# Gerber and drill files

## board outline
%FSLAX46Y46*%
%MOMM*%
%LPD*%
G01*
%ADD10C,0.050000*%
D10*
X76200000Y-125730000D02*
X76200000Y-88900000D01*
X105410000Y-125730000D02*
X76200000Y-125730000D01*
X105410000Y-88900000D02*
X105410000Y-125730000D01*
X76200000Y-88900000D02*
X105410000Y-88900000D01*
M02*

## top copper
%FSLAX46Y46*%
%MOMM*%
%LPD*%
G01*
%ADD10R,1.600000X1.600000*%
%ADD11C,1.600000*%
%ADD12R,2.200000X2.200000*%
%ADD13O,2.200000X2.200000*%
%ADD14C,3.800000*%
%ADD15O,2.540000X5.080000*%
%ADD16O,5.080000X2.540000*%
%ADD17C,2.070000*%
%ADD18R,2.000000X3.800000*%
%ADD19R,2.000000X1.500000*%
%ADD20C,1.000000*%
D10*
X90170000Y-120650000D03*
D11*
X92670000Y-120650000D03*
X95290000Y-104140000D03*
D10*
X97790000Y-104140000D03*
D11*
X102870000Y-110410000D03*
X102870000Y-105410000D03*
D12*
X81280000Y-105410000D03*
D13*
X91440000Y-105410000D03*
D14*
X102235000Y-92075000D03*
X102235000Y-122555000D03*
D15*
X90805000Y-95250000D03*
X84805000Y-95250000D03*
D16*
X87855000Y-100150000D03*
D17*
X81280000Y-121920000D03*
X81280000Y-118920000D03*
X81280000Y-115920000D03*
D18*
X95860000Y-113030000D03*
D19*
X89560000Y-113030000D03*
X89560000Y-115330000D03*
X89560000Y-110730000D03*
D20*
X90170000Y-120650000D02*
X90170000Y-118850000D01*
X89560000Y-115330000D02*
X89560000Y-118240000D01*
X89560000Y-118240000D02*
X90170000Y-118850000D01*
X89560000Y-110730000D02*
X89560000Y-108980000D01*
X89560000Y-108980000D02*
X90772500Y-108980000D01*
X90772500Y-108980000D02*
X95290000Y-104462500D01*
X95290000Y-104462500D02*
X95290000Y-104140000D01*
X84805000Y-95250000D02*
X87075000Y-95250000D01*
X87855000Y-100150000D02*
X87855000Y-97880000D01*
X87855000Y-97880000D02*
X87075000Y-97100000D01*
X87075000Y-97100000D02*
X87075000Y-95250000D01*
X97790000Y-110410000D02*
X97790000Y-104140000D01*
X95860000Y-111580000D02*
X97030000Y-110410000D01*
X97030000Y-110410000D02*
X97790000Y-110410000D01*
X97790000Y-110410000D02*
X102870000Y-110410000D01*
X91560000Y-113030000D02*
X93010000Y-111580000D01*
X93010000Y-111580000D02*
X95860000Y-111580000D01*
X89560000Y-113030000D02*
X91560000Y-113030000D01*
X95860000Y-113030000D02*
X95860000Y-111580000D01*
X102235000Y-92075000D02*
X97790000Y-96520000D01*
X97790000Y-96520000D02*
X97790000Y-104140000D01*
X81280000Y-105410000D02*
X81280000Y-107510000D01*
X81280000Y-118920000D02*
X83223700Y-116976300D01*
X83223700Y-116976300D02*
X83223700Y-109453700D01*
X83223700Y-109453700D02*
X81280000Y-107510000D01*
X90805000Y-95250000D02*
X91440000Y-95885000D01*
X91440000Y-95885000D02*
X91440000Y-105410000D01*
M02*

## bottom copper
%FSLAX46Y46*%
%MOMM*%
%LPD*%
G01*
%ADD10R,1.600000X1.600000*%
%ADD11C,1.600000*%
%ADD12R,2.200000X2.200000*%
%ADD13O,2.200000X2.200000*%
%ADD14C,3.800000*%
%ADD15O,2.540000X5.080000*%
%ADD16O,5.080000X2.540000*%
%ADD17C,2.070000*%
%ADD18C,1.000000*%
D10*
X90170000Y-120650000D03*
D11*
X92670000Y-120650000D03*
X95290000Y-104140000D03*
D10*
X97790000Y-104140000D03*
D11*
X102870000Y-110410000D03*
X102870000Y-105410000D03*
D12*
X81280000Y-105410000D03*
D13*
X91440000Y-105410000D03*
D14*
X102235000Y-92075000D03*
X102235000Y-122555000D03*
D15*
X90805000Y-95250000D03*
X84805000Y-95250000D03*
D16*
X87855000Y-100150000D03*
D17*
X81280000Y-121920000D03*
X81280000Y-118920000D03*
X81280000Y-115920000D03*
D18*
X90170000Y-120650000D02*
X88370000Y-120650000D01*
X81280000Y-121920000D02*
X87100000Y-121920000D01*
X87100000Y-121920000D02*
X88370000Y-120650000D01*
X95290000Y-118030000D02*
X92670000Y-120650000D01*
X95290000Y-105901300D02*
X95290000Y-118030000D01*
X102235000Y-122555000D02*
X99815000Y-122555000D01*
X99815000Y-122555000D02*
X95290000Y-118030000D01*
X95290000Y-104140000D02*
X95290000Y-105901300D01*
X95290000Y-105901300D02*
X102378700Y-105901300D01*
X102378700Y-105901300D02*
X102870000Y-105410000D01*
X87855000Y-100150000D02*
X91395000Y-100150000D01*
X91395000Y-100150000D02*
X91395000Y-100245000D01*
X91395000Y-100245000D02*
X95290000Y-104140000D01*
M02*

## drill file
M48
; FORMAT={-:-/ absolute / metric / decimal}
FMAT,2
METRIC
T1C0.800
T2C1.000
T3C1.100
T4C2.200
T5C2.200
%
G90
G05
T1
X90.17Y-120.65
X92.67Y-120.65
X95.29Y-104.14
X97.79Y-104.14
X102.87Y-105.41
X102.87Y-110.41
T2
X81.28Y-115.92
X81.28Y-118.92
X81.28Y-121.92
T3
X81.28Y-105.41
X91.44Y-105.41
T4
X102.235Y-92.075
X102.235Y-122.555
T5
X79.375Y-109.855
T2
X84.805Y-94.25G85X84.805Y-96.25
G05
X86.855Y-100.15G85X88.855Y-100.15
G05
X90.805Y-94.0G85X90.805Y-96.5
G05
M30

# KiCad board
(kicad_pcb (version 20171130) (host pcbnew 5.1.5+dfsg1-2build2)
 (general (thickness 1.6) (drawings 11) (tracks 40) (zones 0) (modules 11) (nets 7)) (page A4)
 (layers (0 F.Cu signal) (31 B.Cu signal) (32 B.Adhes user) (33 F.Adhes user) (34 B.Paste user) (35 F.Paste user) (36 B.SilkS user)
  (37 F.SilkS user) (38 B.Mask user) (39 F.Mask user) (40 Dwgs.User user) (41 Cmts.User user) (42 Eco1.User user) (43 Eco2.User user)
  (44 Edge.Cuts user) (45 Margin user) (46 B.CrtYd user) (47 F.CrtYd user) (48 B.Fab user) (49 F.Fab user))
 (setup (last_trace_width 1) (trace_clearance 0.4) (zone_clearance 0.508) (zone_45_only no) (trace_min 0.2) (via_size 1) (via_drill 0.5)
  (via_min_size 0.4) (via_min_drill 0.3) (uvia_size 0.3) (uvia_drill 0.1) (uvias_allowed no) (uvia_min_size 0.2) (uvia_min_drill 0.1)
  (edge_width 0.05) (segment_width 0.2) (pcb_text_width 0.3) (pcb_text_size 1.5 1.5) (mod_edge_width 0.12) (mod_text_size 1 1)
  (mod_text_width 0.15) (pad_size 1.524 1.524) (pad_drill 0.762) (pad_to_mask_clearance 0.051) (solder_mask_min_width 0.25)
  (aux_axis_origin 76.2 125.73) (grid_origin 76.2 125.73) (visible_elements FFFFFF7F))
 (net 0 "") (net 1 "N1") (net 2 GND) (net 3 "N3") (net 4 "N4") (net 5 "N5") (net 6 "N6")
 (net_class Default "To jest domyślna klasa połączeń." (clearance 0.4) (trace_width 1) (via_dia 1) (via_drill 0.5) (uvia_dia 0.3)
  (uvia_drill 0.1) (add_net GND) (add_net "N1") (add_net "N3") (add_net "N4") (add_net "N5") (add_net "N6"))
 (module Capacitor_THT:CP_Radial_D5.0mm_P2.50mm (layer F.Cu) (at 90.17 120.65)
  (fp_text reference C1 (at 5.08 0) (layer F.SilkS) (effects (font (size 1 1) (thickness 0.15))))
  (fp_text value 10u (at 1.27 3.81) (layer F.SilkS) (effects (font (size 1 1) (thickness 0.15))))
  (pad 1 thru_hole rect (at 0 0) (size 1.6 1.6) (drill 0.8) (layers *.Cu *.Mask) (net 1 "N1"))
  (pad 2 thru_hole circle (at 2.5 0) (size 1.6 1.6) (drill 0.8) (layers *.Cu *.Mask) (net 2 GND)))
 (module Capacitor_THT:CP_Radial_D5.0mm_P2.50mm (layer F.Cu) (at 97.79 104.14 180)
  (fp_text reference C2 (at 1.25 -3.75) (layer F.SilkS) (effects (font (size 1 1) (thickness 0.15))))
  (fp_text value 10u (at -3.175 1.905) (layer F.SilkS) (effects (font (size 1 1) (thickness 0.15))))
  (pad 2 thru_hole circle (at 2.5 0 180) (size 1.6 1.6) (drill 0.8) (layers *.Cu *.Mask) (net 2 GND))
  (pad 1 thru_hole rect (at 0 0 180) (size 1.6 1.6) (drill 0.8) (layers *.Cu *.Mask) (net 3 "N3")))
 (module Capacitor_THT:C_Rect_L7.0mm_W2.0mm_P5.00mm (layer F.Cu) (at 102.87 110.41 90)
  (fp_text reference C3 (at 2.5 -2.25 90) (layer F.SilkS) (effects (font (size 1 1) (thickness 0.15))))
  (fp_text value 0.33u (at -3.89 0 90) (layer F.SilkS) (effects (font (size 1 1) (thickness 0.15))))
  (pad 1 thru_hole circle (at 0 0 90) (size 1.6 1.6) (drill 0.8) (layers *.Cu *.Mask) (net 3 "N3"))
  (pad 2 thru_hole circle (at 5 0 90) (size 1.6 1.6) (drill 0.8) (layers *.Cu *.Mask) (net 2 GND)))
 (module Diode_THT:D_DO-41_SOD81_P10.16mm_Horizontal (layer F.Cu) (at 81.28 105.41)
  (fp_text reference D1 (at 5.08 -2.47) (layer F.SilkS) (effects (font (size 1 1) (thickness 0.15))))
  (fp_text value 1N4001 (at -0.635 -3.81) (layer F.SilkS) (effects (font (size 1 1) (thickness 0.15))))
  (pad 1 thru_hole rect (at 0 0) (size 2.2 2.2) (drill 1.1) (layers *.Cu *.Mask) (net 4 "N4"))
  (pad 2 thru_hole oval (at 10.16 0) (size 2.2 2.2) (drill 1.1) (layers *.Cu *.Mask) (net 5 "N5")))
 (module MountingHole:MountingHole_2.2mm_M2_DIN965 (layer F.Cu) (at 79.375 109.855)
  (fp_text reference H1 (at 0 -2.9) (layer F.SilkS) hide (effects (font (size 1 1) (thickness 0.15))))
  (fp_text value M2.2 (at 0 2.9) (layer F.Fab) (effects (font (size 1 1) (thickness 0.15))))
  (pad 1 np_thru_hole circle (at 0 0) (size 2.2 2.2) (drill 2.2) (layers *.Cu *.Mask)))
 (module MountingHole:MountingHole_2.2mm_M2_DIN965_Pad (layer F.Cu) (at 102.235 92.075)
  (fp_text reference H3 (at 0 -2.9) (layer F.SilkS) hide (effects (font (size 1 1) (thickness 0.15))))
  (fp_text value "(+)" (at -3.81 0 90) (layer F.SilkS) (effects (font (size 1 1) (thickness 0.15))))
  (pad 1 thru_hole circle (at 0 0) (size 3.8 3.8) (drill 2.2) (layers *.Cu *.Mask) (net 3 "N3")))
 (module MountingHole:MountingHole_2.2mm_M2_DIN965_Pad (layer F.Cu) (at 102.235 122.555)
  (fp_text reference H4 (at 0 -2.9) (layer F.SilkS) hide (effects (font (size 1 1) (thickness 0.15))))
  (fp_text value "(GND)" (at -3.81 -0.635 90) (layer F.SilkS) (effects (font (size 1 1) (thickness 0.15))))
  (pad 1 thru_hole circle (at 0 0) (size 3.8 3.8) (drill 2.2) (layers *.Cu *.Mask) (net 2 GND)))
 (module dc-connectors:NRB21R (layer F.Cu) (at 90.805 95.25 270)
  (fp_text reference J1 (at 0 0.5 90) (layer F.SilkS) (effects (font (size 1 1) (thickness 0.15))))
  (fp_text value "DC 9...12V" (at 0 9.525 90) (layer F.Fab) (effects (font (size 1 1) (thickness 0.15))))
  (pad 1 thru_hole oval (at 0 0 270) (size 5.08 2.54) (drill oval 3.5 1) (layers *.Cu *.Mask) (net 5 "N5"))
  (pad 2 thru_hole oval (at 0 6 270) (size 5.08 2.54) (drill oval 3 1) (layers *.Cu *.Mask) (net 2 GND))
  (pad 3 thru_hole oval (at 4.9 2.95) (size 5.08 2.54) (drill oval 3 1) (layers *.Cu *.Mask) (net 2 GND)))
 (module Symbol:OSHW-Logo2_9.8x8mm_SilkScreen (layer F.Cu) (at 98.425 97.155)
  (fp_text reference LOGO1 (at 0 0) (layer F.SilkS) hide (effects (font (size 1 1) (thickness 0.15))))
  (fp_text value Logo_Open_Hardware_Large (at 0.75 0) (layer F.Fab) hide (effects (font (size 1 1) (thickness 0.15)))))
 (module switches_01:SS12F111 (layer F.Cu) (at 81.28 118.92 90)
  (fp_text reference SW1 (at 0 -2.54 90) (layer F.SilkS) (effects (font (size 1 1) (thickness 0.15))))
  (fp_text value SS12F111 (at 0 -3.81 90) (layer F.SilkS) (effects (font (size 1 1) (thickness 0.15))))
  (pad 1 thru_hole circle (at -3 0 90) (size 2.07 2.07) (drill 1) (layers *.Cu *.Mask) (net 1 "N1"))
  (pad 2 thru_hole circle (at 0 0 90) (size 2.07 2.07) (drill 1) (layers *.Cu *.Mask) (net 4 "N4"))
  (pad 3 thru_hole circle (at 3 0 90) (size 2.07 2.07) (drill 1) (layers *.Cu *.Mask) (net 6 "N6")))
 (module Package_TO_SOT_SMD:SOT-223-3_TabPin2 (layer F.Cu) (at 92.71 113.03)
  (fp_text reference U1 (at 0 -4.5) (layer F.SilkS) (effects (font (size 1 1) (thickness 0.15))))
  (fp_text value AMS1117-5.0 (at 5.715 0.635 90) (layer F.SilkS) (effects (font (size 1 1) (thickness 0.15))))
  (pad 2 smd rect (at 3.15 0) (size 2 3.8) (layers F.Cu F.Paste F.Mask) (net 3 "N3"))
  (pad 2 smd rect (at -3.15 0) (size 2 1.5) (layers F.Cu F.Paste F.Mask) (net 3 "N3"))
  (pad 3 smd rect (at -3.15 2.3) (size 2 1.5) (layers F.Cu F.Paste F.Mask) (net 1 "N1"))
  (pad 1 smd rect (at -3.15 -2.3) (size 2 1.5) (layers F.Cu F.Paste F.Mask) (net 2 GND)))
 (gr_line (start 76.2 125.73) (end 76.2 88.9) (layer Edge.Cuts) (width 0.05))
 (gr_line (start 105.41 125.73) (end 76.2 125.73) (layer Edge.Cuts) (width 0.05))
 (gr_line (start 105.41 88.9) (end 105.41 125.73) (layer Edge.Cuts) (width 0.05))
 (gr_line (start 76.2 88.9) (end 105.41 88.9) (layer Edge.Cuts) (width 0.05))
 (segment (start 90.17 120.65) (end 88.37 120.65) (width 1) (layer B.Cu) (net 1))
 (segment (start 81.28 121.92) (end 87.1 121.92) (width 1) (layer B.Cu) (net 1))
 (segment (start 87.1 121.92) (end 88.37 120.65) (width 1) (layer B.Cu) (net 1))
 (segment (start 90.17 120.65) (end 90.17 118.85) (width 1) (layer F.Cu) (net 1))
 (segment (start 89.56 115.33) (end 89.56 118.24) (width 1) (layer F.Cu) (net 1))
 (segment (start 89.56 118.24) (end 90.17 118.85) (width 1) (layer F.Cu) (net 1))
 (segment (start 95.29 118.03) (end 92.67 120.65) (width 1) (layer B.Cu) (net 2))
 (segment (start 95.29 105.9013) (end 95.29 118.03) (width 1) (layer B.Cu) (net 2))
 (segment (start 102.235 122.555) (end 99.815 122.555) (width 1) (layer B.Cu) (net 2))
 (segment (start 99.815 122.555) (end 95.29 118.03) (width 1) (layer B.Cu) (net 2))
 (segment (start 95.29 104.14) (end 95.29 105.9013) (width 1) (layer B.Cu) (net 2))
 (segment (start 95.29 105.9013) (end 102.3787 105.9013) (width 1) (layer B.Cu) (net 2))
 (segment (start 102.3787 105.9013) (end 102.87 105.41) (width 1) (layer B.Cu) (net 2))
 (segment (start 87.855 100.15) (end 91.395 100.15) (width 1) (layer B.Cu) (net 2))
 (segment (start 91.395 100.15) (end 91.395 100.245) (width 1) (layer B.Cu) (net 2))
 (segment (start 91.395 100.245) (end 95.29 104.14) (width 1) (layer B.Cu) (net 2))
 (segment (start 89.56 110.73) (end 89.56 108.98) (width 1) (layer F.Cu) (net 2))
 (segment (start 89.56 108.98) (end 90.7725 108.98) (width 1) (layer F.Cu) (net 2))
 (segment (start 90.7725 108.98) (end 95.29 104.4625) (width 1) (layer F.Cu) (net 2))
 (segment (start 95.29 104.4625) (end 95.29 104.14) (width 1) (layer F.Cu) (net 2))
 (segment (start 84.805 95.25) (end 87.075 95.25) (width 1) (layer F.Cu) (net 2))
 (segment (start 87.855 100.15) (end 87.855 97.88) (width 1) (layer F.Cu) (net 2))
 (segment (start 87.855 97.88) (end 87.075 97.1) (width 1) (layer F.Cu) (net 2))
 (segment (start 87.075 97.1) (end 87.075 95.25) (width 1) (layer F.Cu) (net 2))
 (segment (start 97.79 110.41) (end 97.79 104.14) (width 1) (layer F.Cu) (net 3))
 (segment (start 95.86 111.58) (end 97.03 110.41) (width 1) (layer F.Cu) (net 3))
 (segment (start 97.03 110.41) (end 97.79 110.41) (width 1) (layer F.Cu) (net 3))
 (segment (start 97.79 110.41) (end 102.87 110.41) (width 1) (layer F.Cu) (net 3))
 (segment (start 91.56 113.03) (end 93.01 111.58) (width 1) (layer F.Cu) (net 3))
 (segment (start 93.01 111.58) (end 95.86 111.58) (width 1) (layer F.Cu) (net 3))
 (segment (start 89.56 113.03) (end 91.56 113.03) (width 1) (layer F.Cu) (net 3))
 (segment (start 95.86 113.03) (end 95.86 111.58) (width 1) (layer F.Cu) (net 3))
 (segment (start 102.235 92.075) (end 97.79 96.52) (width 1) (layer F.Cu) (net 3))
 (segment (start 97.79 96.52) (end 97.79 104.14) (width 1) (layer F.Cu) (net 3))
 (segment (start 81.28 105.41) (end 81.28 107.51) (width 1) (layer F.Cu) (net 4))
 (segment (start 81.28 118.92) (end 83.2237 116.9763) (width 1) (layer F.Cu) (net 4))
 (segment (start 83.2237 116.9763) (end 83.2237 109.4537) (width 1) (layer F.Cu) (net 4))
 (segment (start 83.2237 109.4537) (end 81.28 107.51) (width 1) (layer F.Cu) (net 4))
 (segment (start 90.805 95.25) (end 91.44 95.885) (width 1) (layer F.Cu) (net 5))
 (segment (start 91.44 95.885) (end 91.44 105.41) (width 1) (layer F.Cu) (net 5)))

